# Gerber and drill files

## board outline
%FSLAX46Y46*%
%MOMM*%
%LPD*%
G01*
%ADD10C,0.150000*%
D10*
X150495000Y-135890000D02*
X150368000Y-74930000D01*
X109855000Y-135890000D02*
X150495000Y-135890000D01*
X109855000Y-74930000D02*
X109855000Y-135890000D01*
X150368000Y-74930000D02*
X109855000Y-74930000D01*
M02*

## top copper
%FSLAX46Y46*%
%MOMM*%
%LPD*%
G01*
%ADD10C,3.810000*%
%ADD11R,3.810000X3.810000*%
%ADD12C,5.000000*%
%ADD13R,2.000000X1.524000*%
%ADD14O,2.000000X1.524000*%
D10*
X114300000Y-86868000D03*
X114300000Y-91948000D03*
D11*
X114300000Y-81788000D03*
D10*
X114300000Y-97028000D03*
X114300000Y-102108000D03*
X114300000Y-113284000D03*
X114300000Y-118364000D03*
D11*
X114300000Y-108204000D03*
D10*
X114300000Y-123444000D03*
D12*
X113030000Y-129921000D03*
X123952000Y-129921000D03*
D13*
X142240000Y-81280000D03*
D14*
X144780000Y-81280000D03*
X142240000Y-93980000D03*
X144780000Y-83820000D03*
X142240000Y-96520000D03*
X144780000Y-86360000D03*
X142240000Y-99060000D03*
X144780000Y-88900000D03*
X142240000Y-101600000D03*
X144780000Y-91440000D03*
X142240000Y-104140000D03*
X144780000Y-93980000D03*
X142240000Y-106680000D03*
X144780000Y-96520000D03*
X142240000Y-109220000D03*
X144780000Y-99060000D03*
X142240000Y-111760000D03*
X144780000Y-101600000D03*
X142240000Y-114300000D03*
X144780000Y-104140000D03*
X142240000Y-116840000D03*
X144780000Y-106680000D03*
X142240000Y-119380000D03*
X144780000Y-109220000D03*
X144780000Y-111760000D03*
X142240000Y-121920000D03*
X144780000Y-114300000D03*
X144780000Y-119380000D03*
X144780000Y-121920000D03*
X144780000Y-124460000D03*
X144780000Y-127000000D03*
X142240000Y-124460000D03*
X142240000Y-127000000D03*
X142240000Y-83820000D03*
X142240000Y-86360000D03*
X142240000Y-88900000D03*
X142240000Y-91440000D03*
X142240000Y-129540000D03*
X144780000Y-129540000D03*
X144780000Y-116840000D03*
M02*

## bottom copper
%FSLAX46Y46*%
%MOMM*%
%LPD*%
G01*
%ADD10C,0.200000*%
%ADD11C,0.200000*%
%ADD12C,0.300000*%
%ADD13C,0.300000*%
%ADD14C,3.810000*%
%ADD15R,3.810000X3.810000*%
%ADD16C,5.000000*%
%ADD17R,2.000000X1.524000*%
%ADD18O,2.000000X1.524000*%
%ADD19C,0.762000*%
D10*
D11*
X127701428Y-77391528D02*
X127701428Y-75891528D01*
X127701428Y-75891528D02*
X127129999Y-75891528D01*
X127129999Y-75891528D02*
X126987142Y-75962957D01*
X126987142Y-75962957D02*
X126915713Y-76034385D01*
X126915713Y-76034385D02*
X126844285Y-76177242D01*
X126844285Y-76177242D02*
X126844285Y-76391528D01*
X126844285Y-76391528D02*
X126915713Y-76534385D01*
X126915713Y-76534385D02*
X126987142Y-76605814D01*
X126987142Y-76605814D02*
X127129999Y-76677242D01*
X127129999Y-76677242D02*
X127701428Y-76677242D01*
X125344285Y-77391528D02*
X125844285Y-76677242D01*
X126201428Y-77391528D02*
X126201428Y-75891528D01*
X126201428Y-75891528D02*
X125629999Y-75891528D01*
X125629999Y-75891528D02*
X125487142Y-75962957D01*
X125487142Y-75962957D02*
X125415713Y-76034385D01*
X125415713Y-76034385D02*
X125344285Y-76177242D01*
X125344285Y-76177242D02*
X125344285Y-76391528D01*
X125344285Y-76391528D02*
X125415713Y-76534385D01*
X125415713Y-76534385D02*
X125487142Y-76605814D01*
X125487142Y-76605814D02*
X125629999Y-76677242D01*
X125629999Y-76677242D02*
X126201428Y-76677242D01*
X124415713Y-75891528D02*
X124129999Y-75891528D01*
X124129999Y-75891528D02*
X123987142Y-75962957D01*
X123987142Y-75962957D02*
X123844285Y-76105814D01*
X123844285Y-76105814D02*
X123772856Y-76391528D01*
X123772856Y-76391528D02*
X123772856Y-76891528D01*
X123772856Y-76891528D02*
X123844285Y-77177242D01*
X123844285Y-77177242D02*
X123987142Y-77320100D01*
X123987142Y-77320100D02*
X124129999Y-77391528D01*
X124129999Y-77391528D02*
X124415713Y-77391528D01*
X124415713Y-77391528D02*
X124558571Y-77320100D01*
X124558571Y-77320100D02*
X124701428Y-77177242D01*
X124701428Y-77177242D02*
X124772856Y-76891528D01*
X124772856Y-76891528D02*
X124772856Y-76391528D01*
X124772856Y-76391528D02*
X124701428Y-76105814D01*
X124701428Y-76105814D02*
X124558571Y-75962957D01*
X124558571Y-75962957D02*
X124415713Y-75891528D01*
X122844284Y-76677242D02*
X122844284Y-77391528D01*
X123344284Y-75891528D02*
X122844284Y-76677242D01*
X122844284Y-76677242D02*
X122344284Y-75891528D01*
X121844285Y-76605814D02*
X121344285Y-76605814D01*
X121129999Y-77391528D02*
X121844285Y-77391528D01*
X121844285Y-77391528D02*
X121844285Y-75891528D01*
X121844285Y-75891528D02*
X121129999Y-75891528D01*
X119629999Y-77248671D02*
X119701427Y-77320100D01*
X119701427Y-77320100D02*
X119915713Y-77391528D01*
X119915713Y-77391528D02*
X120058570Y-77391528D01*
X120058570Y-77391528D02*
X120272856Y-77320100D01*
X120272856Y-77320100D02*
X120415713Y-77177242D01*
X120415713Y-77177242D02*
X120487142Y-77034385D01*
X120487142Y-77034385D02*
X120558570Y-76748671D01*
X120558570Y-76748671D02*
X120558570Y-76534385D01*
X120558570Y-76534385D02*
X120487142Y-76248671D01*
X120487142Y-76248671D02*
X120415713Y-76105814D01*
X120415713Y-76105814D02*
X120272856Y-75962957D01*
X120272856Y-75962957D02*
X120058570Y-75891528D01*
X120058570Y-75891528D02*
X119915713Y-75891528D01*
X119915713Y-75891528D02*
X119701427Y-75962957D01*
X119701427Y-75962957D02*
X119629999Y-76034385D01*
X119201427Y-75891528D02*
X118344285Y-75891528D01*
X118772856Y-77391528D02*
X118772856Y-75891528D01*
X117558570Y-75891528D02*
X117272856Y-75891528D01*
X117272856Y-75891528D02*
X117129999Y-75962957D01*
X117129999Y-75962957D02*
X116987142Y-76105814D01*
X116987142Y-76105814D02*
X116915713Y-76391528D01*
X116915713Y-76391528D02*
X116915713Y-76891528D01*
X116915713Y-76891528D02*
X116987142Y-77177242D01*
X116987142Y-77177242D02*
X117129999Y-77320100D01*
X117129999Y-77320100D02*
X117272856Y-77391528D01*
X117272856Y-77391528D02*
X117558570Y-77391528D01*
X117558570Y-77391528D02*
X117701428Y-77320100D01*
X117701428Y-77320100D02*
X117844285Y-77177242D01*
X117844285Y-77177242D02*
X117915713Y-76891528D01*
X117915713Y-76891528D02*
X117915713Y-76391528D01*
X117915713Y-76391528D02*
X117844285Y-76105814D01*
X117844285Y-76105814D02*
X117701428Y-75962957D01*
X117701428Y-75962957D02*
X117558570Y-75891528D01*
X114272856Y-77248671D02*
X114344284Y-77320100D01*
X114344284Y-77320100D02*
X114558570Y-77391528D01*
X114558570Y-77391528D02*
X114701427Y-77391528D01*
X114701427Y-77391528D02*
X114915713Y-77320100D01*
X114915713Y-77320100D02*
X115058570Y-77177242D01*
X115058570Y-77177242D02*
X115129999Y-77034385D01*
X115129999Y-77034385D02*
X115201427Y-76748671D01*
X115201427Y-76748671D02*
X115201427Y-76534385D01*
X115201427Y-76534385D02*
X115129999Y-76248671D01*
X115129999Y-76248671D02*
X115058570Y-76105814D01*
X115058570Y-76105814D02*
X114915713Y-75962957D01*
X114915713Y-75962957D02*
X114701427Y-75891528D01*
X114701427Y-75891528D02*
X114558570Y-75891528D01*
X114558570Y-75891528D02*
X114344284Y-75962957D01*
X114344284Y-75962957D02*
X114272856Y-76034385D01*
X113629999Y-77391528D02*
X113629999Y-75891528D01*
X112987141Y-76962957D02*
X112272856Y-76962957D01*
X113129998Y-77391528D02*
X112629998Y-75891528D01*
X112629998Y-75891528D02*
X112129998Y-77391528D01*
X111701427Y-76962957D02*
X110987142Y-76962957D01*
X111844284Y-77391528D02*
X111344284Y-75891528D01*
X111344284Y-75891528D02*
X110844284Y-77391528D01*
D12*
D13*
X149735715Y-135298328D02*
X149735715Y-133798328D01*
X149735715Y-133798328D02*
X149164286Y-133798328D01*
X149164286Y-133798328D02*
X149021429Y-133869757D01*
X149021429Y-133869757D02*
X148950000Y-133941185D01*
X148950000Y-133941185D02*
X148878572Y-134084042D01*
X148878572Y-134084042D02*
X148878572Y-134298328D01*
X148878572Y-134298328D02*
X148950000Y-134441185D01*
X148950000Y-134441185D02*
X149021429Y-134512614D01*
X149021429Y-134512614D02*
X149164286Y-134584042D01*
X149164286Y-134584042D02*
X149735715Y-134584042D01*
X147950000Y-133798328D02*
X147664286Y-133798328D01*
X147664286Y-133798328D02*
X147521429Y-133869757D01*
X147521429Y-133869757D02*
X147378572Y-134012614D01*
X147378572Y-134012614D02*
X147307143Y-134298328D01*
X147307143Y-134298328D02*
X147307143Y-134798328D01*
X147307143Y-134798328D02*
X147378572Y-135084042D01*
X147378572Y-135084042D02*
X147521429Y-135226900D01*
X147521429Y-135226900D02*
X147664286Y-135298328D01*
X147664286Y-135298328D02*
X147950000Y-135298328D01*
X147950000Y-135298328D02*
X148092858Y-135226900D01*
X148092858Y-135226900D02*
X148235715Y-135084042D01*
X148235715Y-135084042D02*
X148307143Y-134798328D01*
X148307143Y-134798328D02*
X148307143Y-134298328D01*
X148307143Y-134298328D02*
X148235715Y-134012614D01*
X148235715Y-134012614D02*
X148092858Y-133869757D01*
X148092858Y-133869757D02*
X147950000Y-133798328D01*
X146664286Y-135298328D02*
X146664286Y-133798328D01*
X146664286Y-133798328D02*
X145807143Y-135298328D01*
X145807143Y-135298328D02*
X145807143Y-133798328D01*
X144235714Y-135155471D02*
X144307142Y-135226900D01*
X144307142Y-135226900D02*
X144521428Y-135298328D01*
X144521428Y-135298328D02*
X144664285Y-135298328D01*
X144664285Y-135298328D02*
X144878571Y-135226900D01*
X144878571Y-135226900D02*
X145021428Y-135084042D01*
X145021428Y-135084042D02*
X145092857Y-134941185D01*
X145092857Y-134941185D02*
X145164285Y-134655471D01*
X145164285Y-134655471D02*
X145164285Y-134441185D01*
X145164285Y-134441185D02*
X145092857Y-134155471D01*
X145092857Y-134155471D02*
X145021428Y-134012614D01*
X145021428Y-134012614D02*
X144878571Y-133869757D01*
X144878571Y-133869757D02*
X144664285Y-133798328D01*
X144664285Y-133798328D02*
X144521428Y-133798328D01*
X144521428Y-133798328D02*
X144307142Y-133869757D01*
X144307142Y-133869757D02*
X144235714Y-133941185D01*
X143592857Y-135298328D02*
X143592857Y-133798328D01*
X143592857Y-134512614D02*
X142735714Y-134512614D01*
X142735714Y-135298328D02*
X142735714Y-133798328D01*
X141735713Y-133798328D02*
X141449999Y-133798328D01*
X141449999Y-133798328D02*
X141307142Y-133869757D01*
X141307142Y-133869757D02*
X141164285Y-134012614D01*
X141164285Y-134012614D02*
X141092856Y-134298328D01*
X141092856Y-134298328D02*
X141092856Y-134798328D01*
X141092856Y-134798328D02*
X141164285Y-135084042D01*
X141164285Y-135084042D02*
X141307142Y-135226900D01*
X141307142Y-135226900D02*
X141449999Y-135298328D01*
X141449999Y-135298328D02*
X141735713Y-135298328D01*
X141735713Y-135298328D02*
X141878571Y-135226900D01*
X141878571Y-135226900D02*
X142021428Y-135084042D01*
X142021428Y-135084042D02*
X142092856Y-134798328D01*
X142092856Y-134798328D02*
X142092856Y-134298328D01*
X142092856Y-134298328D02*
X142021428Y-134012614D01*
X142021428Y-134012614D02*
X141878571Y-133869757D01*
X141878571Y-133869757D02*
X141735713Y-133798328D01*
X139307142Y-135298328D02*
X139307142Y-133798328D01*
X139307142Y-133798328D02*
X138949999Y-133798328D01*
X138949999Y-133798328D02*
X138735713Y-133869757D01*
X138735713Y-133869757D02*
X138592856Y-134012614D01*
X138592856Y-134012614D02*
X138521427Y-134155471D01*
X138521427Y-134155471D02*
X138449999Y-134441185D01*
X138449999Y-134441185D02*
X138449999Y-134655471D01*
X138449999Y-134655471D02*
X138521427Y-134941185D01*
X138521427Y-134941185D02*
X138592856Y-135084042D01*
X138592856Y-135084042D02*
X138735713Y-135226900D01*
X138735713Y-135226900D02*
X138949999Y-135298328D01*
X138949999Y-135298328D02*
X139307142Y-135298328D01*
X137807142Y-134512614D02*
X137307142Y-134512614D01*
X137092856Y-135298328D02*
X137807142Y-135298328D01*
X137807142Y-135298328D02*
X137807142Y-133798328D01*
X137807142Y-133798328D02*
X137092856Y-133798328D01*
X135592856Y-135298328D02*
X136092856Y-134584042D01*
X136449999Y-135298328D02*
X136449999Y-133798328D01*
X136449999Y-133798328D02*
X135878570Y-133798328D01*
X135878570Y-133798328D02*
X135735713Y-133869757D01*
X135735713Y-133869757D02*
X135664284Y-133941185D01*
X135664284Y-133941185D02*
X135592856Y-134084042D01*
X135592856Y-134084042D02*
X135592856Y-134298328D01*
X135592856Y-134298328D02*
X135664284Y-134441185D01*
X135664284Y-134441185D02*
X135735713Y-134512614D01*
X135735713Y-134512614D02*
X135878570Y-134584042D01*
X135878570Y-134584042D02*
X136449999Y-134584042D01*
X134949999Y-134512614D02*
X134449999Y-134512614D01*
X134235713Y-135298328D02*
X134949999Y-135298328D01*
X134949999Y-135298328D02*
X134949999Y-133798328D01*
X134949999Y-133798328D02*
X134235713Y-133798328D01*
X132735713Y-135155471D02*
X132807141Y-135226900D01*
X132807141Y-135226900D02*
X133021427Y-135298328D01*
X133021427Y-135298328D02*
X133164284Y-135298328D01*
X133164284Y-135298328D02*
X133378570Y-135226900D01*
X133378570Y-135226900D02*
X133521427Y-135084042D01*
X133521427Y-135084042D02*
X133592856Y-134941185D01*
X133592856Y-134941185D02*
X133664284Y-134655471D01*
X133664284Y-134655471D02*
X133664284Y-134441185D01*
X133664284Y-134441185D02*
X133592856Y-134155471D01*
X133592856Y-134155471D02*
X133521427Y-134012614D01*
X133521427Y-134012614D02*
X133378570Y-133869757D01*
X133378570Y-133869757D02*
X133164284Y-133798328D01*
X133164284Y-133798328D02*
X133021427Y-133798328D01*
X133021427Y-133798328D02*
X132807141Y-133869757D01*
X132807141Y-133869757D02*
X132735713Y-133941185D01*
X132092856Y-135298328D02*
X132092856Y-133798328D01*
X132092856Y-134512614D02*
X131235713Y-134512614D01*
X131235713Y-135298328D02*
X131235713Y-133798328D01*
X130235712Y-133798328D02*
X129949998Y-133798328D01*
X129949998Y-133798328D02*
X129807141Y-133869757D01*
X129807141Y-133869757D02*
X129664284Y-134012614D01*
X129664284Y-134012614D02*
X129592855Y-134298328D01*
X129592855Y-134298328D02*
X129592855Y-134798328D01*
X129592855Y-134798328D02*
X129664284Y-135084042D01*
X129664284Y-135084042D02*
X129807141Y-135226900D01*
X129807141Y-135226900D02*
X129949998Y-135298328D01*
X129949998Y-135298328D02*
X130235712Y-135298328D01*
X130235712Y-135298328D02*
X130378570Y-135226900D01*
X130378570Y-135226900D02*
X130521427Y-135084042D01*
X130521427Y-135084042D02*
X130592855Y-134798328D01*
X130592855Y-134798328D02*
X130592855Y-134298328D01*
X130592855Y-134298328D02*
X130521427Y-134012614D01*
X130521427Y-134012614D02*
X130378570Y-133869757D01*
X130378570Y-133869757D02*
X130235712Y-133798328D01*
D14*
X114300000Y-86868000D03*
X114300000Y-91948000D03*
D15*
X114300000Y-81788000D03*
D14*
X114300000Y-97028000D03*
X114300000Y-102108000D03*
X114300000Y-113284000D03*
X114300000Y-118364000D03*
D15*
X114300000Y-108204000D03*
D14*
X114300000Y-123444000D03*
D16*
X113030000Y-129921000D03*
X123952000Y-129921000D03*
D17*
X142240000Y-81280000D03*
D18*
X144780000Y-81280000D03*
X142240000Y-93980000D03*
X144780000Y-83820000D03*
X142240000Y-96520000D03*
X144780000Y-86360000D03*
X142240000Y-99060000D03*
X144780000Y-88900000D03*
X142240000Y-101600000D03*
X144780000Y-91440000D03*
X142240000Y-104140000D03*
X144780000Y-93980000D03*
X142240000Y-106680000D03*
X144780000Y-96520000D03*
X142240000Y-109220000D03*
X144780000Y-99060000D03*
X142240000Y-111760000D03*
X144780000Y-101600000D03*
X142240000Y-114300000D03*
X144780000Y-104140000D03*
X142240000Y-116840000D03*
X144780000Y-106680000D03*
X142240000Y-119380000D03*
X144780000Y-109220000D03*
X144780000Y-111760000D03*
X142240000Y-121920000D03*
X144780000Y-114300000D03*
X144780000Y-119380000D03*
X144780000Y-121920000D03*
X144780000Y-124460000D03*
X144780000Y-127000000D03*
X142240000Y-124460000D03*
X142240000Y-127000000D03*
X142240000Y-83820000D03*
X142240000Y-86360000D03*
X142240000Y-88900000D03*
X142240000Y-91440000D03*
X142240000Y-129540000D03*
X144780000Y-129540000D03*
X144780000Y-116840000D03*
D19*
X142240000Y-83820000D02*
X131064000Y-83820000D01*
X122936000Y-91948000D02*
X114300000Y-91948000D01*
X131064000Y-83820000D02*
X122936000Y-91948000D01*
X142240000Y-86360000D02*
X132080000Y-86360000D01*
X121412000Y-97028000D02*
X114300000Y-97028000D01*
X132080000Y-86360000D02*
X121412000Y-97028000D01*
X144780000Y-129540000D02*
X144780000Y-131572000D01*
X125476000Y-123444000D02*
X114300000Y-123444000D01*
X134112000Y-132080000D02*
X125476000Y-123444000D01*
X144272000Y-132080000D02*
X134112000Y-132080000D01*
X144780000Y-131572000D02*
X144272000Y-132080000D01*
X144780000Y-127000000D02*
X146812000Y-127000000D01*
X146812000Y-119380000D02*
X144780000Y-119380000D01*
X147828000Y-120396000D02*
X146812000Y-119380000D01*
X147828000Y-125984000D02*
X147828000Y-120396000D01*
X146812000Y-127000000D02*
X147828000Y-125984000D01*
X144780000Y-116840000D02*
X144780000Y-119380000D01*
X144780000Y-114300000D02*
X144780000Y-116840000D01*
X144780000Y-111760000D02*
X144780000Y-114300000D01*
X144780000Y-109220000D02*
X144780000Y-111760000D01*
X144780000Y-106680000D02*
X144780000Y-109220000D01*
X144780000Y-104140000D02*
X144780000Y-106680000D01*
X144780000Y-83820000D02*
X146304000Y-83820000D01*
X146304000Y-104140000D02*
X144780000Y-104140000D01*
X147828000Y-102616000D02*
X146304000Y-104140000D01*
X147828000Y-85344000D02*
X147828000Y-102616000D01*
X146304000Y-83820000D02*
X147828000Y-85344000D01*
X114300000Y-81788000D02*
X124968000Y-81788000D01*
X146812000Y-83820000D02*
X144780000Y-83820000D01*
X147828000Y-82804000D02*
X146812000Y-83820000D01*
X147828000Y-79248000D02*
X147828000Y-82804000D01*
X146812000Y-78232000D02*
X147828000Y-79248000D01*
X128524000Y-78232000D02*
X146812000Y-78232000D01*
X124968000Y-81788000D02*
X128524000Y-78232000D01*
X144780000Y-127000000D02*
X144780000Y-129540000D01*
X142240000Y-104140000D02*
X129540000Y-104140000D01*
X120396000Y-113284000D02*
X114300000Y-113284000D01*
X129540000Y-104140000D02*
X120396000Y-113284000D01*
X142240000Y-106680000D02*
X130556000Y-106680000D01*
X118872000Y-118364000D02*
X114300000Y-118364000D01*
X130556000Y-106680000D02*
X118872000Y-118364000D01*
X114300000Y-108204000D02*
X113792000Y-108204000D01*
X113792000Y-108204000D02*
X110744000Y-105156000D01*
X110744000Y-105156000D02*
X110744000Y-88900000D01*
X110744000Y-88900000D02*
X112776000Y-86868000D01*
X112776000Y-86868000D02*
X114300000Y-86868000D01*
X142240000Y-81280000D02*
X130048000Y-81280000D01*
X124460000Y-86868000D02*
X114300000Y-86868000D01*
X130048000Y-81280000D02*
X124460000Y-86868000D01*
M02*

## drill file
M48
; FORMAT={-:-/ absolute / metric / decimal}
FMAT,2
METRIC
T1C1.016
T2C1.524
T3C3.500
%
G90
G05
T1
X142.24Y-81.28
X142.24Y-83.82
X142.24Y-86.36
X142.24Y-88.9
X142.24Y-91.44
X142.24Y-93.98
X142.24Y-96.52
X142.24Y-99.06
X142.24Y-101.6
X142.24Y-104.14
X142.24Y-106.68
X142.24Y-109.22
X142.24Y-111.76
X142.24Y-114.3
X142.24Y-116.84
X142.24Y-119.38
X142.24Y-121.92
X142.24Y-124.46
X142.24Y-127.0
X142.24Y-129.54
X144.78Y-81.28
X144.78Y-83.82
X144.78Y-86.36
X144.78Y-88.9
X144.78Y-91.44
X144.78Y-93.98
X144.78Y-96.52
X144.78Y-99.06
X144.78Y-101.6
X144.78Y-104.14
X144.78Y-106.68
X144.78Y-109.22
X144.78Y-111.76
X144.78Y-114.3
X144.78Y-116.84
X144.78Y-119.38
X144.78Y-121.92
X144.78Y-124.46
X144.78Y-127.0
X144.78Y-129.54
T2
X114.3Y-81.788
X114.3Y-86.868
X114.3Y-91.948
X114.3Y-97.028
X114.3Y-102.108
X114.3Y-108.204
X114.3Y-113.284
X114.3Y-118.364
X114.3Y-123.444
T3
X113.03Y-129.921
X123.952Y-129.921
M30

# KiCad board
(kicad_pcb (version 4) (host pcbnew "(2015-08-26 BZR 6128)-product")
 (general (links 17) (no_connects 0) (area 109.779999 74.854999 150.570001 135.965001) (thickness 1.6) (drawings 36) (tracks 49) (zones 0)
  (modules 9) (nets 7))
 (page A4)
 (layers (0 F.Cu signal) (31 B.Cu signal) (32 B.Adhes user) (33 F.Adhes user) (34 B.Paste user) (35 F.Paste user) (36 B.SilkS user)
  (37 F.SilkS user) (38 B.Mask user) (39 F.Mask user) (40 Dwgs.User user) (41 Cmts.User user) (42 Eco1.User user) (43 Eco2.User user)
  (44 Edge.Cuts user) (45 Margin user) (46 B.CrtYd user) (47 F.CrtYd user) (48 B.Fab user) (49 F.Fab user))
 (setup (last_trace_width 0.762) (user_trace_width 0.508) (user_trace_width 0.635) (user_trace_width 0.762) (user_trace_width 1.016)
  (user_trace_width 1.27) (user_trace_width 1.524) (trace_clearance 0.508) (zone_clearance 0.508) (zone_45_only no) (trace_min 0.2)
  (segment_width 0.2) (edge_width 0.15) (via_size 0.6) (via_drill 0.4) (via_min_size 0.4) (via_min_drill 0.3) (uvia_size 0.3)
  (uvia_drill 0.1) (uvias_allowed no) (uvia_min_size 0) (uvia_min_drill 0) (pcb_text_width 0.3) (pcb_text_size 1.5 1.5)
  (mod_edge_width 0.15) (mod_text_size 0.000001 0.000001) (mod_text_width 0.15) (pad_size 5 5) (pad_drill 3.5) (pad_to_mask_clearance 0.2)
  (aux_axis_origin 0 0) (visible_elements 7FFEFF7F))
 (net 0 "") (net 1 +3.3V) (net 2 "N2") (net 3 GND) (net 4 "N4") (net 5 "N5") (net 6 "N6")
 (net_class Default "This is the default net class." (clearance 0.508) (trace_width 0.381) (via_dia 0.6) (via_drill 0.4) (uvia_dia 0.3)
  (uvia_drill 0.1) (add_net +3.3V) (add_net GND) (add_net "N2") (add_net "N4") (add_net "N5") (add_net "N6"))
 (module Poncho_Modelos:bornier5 (layer F.Cu) (at 114.3 91.948 270)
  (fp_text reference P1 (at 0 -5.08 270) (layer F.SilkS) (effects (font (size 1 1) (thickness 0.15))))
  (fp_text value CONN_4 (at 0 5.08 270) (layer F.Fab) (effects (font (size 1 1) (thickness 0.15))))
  (pad 2 thru_hole circle (at -5.08 0 270) (size 3.81 3.81) (drill 1.524) (layers *.Cu *.Mask F.SilkS) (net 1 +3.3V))
  (pad 3 thru_hole circle (at 0 0 270) (size 3.81 3.81) (drill 1.524) (layers *.Cu *.Mask F.SilkS) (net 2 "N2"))
  (pad 1 thru_hole rect (at -10.16 0 270) (size 3.81 3.81) (drill 1.524) (layers *.Cu *.Mask F.SilkS) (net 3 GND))
  (pad 4 thru_hole circle (at 5.08 0 270) (size 3.81 3.81) (drill 1.524) (layers *.Cu *.Mask F.SilkS) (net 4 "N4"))
  (pad 5 thru_hole circle (at 10.16 0 270) (size 3.81 3.81) (drill 1.524) (layers *.Cu *.Mask F.SilkS)))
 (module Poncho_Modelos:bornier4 (layer F.Cu) (at 114.3 115.824 270)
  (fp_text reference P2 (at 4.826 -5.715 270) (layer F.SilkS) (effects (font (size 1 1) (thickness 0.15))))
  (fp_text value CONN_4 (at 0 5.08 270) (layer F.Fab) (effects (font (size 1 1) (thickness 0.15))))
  (pad 2 thru_hole circle (at -2.54 0 270) (size 3.81 3.81) (drill 1.524) (layers *.Cu *.Mask F.SilkS) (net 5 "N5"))
  (pad 3 thru_hole circle (at 2.54 0 270) (size 3.81 3.81) (drill 1.524) (layers *.Cu *.Mask F.SilkS) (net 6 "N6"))
  (pad 1 thru_hole rect (at -7.62 0 270) (size 3.81 3.81) (drill 1.524) (layers *.Cu *.Mask F.SilkS) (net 1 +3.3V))
  (pad 4 thru_hole circle (at 7.62 0 270) (size 3.81 3.81) (drill 1.524) (layers *.Cu *.Mask F.SilkS) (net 3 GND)))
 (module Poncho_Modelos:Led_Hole (layer F.Cu) (at 113.03 129.921)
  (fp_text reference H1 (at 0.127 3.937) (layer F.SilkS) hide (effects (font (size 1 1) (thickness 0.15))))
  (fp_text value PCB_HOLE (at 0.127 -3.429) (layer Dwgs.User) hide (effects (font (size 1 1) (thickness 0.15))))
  (pad 1 thru_hole circle (at 0 0) (size 5 5) (drill 3.5) (layers *.Cu *.Mask F.SilkS)))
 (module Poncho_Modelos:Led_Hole (layer F.Cu) (at 123.952 129.921)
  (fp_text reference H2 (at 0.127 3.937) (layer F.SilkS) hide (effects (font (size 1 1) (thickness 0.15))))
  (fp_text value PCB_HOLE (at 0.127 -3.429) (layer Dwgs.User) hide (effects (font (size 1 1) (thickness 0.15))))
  (pad 1 thru_hole circle (at 0 0) (size 5 5) (drill 3.5) (layers *.Cu *.Mask F.SilkS)))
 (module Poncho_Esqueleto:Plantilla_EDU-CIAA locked (layer F.Cu) (at 142.24 81.28)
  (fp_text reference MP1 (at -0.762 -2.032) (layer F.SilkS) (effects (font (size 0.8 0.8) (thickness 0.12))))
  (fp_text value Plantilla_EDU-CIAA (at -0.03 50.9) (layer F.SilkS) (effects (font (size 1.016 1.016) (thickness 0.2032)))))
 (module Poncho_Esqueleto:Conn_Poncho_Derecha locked (layer F.Cu) (at 142.24 81.28)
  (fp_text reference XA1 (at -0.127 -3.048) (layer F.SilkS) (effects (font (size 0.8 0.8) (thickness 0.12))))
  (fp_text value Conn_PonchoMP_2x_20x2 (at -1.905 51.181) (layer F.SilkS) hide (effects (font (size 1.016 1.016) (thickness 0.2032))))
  (pad 1 thru_hole rect (at 0 0 270) (size 1.524 2) (drill 1.016) (layers *.Cu *.Mask F.SilkS) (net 1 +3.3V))
  (pad 2 thru_hole oval (at 2.54 0 270) (size 1.524 2) (drill 1.016) (layers *.Cu *.Mask F.SilkS))
  (pad 11 thru_hole oval (at 0 12.7 270) (size 1.524 2) (drill 1.016) (layers *.Cu *.Mask F.SilkS))
  (pad 4 thru_hole oval (at 2.54 2.54 270) (size 1.524 2) (drill 1.016) (layers *.Cu *.Mask F.SilkS) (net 3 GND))
  (pad 13 thru_hole oval (at 0 15.24 270) (size 1.524 2) (drill 1.016) (layers *.Cu *.Mask F.SilkS))
  (pad 6 thru_hole oval (at 2.54 5.08 270) (size 1.524 2) (drill 1.016) (layers *.Cu *.Mask F.SilkS))
  (pad 15 thru_hole oval (at 0 17.78 270) (size 1.524 2) (drill 1.016) (layers *.Cu *.Mask F.SilkS))
  (pad 8 thru_hole oval (at 2.54 7.62 270) (size 1.524 2) (drill 1.016) (layers *.Cu *.Mask F.SilkS))
  (pad 17 thru_hole oval (at 0 20.32 270) (size 1.524 2) (drill 1.016) (layers *.Cu *.Mask F.SilkS))
  (pad 10 thru_hole oval (at 2.54 10.16 270) (size 1.524 2) (drill 1.016) (layers *.Cu *.Mask F.SilkS))
  (pad 19 thru_hole oval (at 0 22.86 270) (size 1.524 2) (drill 1.016) (layers *.Cu *.Mask F.SilkS) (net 5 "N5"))
  (pad 12 thru_hole oval (at 2.54 12.7 270) (size 1.524 2) (drill 1.016) (layers *.Cu *.Mask F.SilkS))
  (pad 21 thru_hole oval (at 0 25.4 270) (size 1.524 2) (drill 1.016) (layers *.Cu *.Mask F.SilkS) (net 6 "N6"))
  (pad 14 thru_hole oval (at 2.54 15.24 270) (size 1.524 2) (drill 1.016) (layers *.Cu *.Mask F.SilkS))
  (pad 23 thru_hole oval (at 0 27.94 270) (size 1.524 2) (drill 1.016) (layers *.Cu *.Mask F.SilkS))
  (pad 16 thru_hole oval (at 2.54 17.78 270) (size 1.524 2) (drill 1.016) (layers *.Cu *.Mask F.SilkS))
  (pad 25 thru_hole oval (at 0 30.48 270) (size 1.524 2) (drill 1.016) (layers *.Cu *.Mask F.SilkS))
  (pad 18 thru_hole oval (at 2.54 20.32 270) (size 1.524 2) (drill 1.016) (layers *.Cu *.Mask F.SilkS))
  (pad 27 thru_hole oval (at 0 33.02 270) (size 1.524 2) (drill 1.016) (layers *.Cu *.Mask F.SilkS))
  (pad 20 thru_hole oval (at 2.54 22.86 270) (size 1.524 2) (drill 1.016) (layers *.Cu *.Mask F.SilkS) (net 3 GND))
  (pad 29 thru_hole oval (at 0 35.56 270) (size 1.524 2) (drill 1.016) (layers *.Cu *.Mask F.SilkS))
  (pad 22 thru_hole oval (at 2.54 25.4 270) (size 1.524 2) (drill 1.016) (layers *.Cu *.Mask F.SilkS) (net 3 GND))
  (pad 31 thru_hole oval (at 0 38.1 270) (size 1.524 2) (drill 1.016) (layers *.Cu *.Mask F.SilkS))
  (pad 24 thru_hole oval (at 2.54 27.94 270) (size 1.524 2) (drill 1.016) (layers *.Cu *.Mask F.SilkS) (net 3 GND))
  (pad 26 thru_hole oval (at 2.54 30.48 270) (size 1.524 2) (drill 1.016) (layers *.Cu *.Mask F.SilkS) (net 3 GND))
  (pad 33 thru_hole oval (at 0 40.64 270) (size 1.524 2) (drill 1.016) (layers *.Cu *.Mask F.SilkS))
  (pad 28 thru_hole oval (at 2.54 33.02 270) (size 1.524 2) (drill 1.016) (layers *.Cu *.Mask F.SilkS) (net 3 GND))
  (pad 32 thru_hole oval (at 2.54 38.1 270) (size 1.524 2) (drill 1.016) (layers *.Cu *.Mask F.SilkS) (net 3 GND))
  (pad 34 thru_hole oval (at 2.54 40.64 270) (size 1.524 2) (drill 1.016) (layers *.Cu *.Mask F.SilkS))
  (pad 36 thru_hole oval (at 2.54 43.18 270) (size 1.524 2) (drill 1.016) (layers *.Cu *.Mask F.SilkS))
  (pad 38 thru_hole oval (at 2.54 45.72 270) (size 1.524 2) (drill 1.016) (layers *.Cu *.Mask F.SilkS) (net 3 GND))
  (pad 35 thru_hole oval (at 0 43.18 270) (size 1.524 2) (drill 1.016) (layers *.Cu *.Mask F.SilkS))
  (pad 37 thru_hole oval (at 0 45.72 270) (size 1.524 2) (drill 1.016) (layers *.Cu *.Mask F.SilkS))
  (pad 3 thru_hole oval (at 0 2.54 270) (size 1.524 2) (drill 1.016) (layers *.Cu *.Mask F.SilkS) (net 2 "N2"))
  (pad 5 thru_hole oval (at 0 5.08 270) (size 1.524 2) (drill 1.016) (layers *.Cu *.Mask F.SilkS) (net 4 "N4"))
  (pad 7 thru_hole oval (at 0 7.62 270) (size 1.524 2) (drill 1.016) (layers *.Cu *.Mask F.SilkS))
  (pad 9 thru_hole oval (at 0 10.16 270) (size 1.524 2) (drill 1.016) (layers *.Cu *.Mask F.SilkS))
  (pad 39 thru_hole oval (at 0 48.26 270) (size 1.524 2) (drill 1.016) (layers *.Cu *.Mask F.SilkS))
  (pad 40 thru_hole oval (at 2.54 48.26 270) (size 1.524 2) (drill 1.016) (layers *.Cu *.Mask F.SilkS) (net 3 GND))
  (pad 30 thru_hole oval (at 2.54 35.56 270) (size 1.524 2) (drill 1.016) (layers *.Cu *.Mask F.SilkS) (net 3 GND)))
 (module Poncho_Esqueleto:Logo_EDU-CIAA (layer F.Cu) (at 127.635 108.585)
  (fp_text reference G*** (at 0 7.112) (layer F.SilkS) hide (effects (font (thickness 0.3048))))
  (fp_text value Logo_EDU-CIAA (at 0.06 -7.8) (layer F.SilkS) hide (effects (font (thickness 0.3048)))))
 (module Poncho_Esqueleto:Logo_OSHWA (layer F.Cu) (at 128.905 96.52)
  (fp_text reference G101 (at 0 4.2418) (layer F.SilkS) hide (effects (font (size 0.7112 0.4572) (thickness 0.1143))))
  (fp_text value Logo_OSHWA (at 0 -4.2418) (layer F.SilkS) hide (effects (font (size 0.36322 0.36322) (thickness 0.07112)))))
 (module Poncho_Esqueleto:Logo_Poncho (layer F.Cu) (at 128.905 83.82)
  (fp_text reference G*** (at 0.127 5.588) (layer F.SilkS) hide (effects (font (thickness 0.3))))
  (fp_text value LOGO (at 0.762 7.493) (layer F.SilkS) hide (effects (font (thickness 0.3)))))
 (gr_line (start 150.495 135.89) (end 150.368 74.93) (angle 90) (layer Edge.Cuts) (width 0.15))
 (gr_line (start 109.855 135.89) (end 150.495 135.89) (angle 90) (layer Edge.Cuts) (width 0.15))
 (gr_line (start 109.855 74.93) (end 109.855 135.89) (angle 90) (layer Edge.Cuts) (width 0.15))
 (gr_line (start 150.368 74.93) (end 109.855 74.93) (angle 90) (layer Edge.Cuts) (width 0.15))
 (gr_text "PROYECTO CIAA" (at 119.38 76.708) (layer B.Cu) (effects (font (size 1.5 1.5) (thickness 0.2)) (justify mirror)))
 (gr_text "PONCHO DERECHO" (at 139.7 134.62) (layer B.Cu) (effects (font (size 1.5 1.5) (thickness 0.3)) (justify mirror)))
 (segment (start 142.24 83.82) (end 131.064 83.82) (width 0.762) (layer B.Cu) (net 2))
 (segment (start 122.936 91.948) (end 114.3 91.948) (width 0.762) (layer B.Cu) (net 2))
 (segment (start 131.064 83.82) (end 122.936 91.948) (width 0.762) (layer B.Cu) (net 2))
 (segment (start 142.24 86.36) (end 132.08 86.36) (width 0.762) (layer B.Cu) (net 4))
 (segment (start 121.412 97.028) (end 114.3 97.028) (width 0.762) (layer B.Cu) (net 4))
 (segment (start 132.08 86.36) (end 121.412 97.028) (width 0.762) (layer B.Cu) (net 4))
 (segment (start 144.78 129.54) (end 144.78 131.572) (width 0.762) (layer B.Cu) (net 3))
 (segment (start 125.476 123.444) (end 114.3 123.444) (width 0.762) (layer B.Cu) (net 3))
 (segment (start 134.112 132.08) (end 125.476 123.444) (width 0.762) (layer B.Cu) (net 3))
 (segment (start 144.272 132.08) (end 134.112 132.08) (width 0.762) (layer B.Cu) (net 3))
 (segment (start 144.78 131.572) (end 144.272 132.08) (width 0.762) (layer B.Cu) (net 3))
 (segment (start 144.78 127) (end 146.812 127) (width 0.762) (layer B.Cu) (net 3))
 (segment (start 146.812 119.38) (end 144.78 119.38) (width 0.762) (layer B.Cu) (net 3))
 (segment (start 147.828 120.396) (end 146.812 119.38) (width 0.762) (layer B.Cu) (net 3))
 (segment (start 147.828 125.984) (end 147.828 120.396) (width 0.762) (layer B.Cu) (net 3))
 (segment (start 146.812 127) (end 147.828 125.984) (width 0.762) (layer B.Cu) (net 3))
 (segment (start 144.78 116.84) (end 144.78 119.38) (width 0.762) (layer B.Cu) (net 3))
 (segment (start 144.78 114.3) (end 144.78 116.84) (width 0.762) (layer B.Cu) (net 3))
 (segment (start 144.78 111.76) (end 144.78 114.3) (width 0.762) (layer B.Cu) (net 3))
 (segment (start 144.78 109.22) (end 144.78 111.76) (width 0.762) (layer B.Cu) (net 3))
 (segment (start 144.78 106.68) (end 144.78 109.22) (width 0.762) (layer B.Cu) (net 3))
 (segment (start 144.78 104.14) (end 144.78 106.68) (width 0.762) (layer B.Cu) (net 3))
 (segment (start 144.78 83.82) (end 146.304 83.82) (width 0.762) (layer B.Cu) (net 3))
 (segment (start 146.304 104.14) (end 144.78 104.14) (width 0.762) (layer B.Cu) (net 3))
 (segment (start 147.828 102.616) (end 146.304 104.14) (width 0.762) (layer B.Cu) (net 3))
 (segment (start 147.828 85.344) (end 147.828 102.616) (width 0.762) (layer B.Cu) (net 3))
 (segment (start 146.304 83.82) (end 147.828 85.344) (width 0.762) (layer B.Cu) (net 3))
 (segment (start 114.3 81.788) (end 124.968 81.788) (width 0.762) (layer B.Cu) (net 3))
 (segment (start 146.812 83.82) (end 144.78 83.82) (width 0.762) (layer B.Cu) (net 3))
 (segment (start 147.828 82.804) (end 146.812 83.82) (width 0.762) (layer B.Cu) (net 3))
 (segment (start 147.828 79.248) (end 147.828 82.804) (width 0.762) (layer B.Cu) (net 3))
 (segment (start 146.812 78.232) (end 147.828 79.248) (width 0.762) (layer B.Cu) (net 3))
 (segment (start 128.524 78.232) (end 146.812 78.232) (width 0.762) (layer B.Cu) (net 3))
 (segment (start 124.968 81.788) (end 128.524 78.232) (width 0.762) (layer B.Cu) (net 3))
 (segment (start 144.78 127) (end 144.78 129.54) (width 0.762) (layer B.Cu) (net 3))
 (segment (start 142.24 104.14) (end 129.54 104.14) (width 0.762) (layer B.Cu) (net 5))
 (segment (start 120.396 113.284) (end 114.3 113.284) (width 0.762) (layer B.Cu) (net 5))
 (segment (start 129.54 104.14) (end 120.396 113.284) (width 0.762) (layer B.Cu) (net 5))
 (segment (start 142.24 106.68) (end 130.556 106.68) (width 0.762) (layer B.Cu) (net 6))
 (segment (start 118.872 118.364) (end 114.3 118.364) (width 0.762) (layer B.Cu) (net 6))
 (segment (start 130.556 106.68) (end 118.872 118.364) (width 0.762) (layer B.Cu) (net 6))
 (segment (start 114.3 108.204) (end 113.792 108.204) (width 0.762) (layer B.Cu) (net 1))
 (segment (start 113.792 108.204) (end 110.744 105.156) (width 0.762) (layer B.Cu) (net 1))
 (segment (start 110.744 105.156) (end 110.744 88.9) (width 0.762) (layer B.Cu) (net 1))
 (segment (start 110.744 88.9) (end 112.776 86.868) (width 0.762) (layer B.Cu) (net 1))
 (segment (start 112.776 86.868) (end 114.3 86.868) (width 0.762) (layer B.Cu) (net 1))
 (segment (start 142.24 81.28) (end 130.048 81.28) (width 0.762) (layer B.Cu) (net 1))
 (segment (start 124.46 86.868) (end 114.3 86.868) (width 0.762) (layer B.Cu) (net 1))
 (segment (start 130.048 81.28) (end 124.46 86.868) (width 0.762) (layer B.Cu) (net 1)))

